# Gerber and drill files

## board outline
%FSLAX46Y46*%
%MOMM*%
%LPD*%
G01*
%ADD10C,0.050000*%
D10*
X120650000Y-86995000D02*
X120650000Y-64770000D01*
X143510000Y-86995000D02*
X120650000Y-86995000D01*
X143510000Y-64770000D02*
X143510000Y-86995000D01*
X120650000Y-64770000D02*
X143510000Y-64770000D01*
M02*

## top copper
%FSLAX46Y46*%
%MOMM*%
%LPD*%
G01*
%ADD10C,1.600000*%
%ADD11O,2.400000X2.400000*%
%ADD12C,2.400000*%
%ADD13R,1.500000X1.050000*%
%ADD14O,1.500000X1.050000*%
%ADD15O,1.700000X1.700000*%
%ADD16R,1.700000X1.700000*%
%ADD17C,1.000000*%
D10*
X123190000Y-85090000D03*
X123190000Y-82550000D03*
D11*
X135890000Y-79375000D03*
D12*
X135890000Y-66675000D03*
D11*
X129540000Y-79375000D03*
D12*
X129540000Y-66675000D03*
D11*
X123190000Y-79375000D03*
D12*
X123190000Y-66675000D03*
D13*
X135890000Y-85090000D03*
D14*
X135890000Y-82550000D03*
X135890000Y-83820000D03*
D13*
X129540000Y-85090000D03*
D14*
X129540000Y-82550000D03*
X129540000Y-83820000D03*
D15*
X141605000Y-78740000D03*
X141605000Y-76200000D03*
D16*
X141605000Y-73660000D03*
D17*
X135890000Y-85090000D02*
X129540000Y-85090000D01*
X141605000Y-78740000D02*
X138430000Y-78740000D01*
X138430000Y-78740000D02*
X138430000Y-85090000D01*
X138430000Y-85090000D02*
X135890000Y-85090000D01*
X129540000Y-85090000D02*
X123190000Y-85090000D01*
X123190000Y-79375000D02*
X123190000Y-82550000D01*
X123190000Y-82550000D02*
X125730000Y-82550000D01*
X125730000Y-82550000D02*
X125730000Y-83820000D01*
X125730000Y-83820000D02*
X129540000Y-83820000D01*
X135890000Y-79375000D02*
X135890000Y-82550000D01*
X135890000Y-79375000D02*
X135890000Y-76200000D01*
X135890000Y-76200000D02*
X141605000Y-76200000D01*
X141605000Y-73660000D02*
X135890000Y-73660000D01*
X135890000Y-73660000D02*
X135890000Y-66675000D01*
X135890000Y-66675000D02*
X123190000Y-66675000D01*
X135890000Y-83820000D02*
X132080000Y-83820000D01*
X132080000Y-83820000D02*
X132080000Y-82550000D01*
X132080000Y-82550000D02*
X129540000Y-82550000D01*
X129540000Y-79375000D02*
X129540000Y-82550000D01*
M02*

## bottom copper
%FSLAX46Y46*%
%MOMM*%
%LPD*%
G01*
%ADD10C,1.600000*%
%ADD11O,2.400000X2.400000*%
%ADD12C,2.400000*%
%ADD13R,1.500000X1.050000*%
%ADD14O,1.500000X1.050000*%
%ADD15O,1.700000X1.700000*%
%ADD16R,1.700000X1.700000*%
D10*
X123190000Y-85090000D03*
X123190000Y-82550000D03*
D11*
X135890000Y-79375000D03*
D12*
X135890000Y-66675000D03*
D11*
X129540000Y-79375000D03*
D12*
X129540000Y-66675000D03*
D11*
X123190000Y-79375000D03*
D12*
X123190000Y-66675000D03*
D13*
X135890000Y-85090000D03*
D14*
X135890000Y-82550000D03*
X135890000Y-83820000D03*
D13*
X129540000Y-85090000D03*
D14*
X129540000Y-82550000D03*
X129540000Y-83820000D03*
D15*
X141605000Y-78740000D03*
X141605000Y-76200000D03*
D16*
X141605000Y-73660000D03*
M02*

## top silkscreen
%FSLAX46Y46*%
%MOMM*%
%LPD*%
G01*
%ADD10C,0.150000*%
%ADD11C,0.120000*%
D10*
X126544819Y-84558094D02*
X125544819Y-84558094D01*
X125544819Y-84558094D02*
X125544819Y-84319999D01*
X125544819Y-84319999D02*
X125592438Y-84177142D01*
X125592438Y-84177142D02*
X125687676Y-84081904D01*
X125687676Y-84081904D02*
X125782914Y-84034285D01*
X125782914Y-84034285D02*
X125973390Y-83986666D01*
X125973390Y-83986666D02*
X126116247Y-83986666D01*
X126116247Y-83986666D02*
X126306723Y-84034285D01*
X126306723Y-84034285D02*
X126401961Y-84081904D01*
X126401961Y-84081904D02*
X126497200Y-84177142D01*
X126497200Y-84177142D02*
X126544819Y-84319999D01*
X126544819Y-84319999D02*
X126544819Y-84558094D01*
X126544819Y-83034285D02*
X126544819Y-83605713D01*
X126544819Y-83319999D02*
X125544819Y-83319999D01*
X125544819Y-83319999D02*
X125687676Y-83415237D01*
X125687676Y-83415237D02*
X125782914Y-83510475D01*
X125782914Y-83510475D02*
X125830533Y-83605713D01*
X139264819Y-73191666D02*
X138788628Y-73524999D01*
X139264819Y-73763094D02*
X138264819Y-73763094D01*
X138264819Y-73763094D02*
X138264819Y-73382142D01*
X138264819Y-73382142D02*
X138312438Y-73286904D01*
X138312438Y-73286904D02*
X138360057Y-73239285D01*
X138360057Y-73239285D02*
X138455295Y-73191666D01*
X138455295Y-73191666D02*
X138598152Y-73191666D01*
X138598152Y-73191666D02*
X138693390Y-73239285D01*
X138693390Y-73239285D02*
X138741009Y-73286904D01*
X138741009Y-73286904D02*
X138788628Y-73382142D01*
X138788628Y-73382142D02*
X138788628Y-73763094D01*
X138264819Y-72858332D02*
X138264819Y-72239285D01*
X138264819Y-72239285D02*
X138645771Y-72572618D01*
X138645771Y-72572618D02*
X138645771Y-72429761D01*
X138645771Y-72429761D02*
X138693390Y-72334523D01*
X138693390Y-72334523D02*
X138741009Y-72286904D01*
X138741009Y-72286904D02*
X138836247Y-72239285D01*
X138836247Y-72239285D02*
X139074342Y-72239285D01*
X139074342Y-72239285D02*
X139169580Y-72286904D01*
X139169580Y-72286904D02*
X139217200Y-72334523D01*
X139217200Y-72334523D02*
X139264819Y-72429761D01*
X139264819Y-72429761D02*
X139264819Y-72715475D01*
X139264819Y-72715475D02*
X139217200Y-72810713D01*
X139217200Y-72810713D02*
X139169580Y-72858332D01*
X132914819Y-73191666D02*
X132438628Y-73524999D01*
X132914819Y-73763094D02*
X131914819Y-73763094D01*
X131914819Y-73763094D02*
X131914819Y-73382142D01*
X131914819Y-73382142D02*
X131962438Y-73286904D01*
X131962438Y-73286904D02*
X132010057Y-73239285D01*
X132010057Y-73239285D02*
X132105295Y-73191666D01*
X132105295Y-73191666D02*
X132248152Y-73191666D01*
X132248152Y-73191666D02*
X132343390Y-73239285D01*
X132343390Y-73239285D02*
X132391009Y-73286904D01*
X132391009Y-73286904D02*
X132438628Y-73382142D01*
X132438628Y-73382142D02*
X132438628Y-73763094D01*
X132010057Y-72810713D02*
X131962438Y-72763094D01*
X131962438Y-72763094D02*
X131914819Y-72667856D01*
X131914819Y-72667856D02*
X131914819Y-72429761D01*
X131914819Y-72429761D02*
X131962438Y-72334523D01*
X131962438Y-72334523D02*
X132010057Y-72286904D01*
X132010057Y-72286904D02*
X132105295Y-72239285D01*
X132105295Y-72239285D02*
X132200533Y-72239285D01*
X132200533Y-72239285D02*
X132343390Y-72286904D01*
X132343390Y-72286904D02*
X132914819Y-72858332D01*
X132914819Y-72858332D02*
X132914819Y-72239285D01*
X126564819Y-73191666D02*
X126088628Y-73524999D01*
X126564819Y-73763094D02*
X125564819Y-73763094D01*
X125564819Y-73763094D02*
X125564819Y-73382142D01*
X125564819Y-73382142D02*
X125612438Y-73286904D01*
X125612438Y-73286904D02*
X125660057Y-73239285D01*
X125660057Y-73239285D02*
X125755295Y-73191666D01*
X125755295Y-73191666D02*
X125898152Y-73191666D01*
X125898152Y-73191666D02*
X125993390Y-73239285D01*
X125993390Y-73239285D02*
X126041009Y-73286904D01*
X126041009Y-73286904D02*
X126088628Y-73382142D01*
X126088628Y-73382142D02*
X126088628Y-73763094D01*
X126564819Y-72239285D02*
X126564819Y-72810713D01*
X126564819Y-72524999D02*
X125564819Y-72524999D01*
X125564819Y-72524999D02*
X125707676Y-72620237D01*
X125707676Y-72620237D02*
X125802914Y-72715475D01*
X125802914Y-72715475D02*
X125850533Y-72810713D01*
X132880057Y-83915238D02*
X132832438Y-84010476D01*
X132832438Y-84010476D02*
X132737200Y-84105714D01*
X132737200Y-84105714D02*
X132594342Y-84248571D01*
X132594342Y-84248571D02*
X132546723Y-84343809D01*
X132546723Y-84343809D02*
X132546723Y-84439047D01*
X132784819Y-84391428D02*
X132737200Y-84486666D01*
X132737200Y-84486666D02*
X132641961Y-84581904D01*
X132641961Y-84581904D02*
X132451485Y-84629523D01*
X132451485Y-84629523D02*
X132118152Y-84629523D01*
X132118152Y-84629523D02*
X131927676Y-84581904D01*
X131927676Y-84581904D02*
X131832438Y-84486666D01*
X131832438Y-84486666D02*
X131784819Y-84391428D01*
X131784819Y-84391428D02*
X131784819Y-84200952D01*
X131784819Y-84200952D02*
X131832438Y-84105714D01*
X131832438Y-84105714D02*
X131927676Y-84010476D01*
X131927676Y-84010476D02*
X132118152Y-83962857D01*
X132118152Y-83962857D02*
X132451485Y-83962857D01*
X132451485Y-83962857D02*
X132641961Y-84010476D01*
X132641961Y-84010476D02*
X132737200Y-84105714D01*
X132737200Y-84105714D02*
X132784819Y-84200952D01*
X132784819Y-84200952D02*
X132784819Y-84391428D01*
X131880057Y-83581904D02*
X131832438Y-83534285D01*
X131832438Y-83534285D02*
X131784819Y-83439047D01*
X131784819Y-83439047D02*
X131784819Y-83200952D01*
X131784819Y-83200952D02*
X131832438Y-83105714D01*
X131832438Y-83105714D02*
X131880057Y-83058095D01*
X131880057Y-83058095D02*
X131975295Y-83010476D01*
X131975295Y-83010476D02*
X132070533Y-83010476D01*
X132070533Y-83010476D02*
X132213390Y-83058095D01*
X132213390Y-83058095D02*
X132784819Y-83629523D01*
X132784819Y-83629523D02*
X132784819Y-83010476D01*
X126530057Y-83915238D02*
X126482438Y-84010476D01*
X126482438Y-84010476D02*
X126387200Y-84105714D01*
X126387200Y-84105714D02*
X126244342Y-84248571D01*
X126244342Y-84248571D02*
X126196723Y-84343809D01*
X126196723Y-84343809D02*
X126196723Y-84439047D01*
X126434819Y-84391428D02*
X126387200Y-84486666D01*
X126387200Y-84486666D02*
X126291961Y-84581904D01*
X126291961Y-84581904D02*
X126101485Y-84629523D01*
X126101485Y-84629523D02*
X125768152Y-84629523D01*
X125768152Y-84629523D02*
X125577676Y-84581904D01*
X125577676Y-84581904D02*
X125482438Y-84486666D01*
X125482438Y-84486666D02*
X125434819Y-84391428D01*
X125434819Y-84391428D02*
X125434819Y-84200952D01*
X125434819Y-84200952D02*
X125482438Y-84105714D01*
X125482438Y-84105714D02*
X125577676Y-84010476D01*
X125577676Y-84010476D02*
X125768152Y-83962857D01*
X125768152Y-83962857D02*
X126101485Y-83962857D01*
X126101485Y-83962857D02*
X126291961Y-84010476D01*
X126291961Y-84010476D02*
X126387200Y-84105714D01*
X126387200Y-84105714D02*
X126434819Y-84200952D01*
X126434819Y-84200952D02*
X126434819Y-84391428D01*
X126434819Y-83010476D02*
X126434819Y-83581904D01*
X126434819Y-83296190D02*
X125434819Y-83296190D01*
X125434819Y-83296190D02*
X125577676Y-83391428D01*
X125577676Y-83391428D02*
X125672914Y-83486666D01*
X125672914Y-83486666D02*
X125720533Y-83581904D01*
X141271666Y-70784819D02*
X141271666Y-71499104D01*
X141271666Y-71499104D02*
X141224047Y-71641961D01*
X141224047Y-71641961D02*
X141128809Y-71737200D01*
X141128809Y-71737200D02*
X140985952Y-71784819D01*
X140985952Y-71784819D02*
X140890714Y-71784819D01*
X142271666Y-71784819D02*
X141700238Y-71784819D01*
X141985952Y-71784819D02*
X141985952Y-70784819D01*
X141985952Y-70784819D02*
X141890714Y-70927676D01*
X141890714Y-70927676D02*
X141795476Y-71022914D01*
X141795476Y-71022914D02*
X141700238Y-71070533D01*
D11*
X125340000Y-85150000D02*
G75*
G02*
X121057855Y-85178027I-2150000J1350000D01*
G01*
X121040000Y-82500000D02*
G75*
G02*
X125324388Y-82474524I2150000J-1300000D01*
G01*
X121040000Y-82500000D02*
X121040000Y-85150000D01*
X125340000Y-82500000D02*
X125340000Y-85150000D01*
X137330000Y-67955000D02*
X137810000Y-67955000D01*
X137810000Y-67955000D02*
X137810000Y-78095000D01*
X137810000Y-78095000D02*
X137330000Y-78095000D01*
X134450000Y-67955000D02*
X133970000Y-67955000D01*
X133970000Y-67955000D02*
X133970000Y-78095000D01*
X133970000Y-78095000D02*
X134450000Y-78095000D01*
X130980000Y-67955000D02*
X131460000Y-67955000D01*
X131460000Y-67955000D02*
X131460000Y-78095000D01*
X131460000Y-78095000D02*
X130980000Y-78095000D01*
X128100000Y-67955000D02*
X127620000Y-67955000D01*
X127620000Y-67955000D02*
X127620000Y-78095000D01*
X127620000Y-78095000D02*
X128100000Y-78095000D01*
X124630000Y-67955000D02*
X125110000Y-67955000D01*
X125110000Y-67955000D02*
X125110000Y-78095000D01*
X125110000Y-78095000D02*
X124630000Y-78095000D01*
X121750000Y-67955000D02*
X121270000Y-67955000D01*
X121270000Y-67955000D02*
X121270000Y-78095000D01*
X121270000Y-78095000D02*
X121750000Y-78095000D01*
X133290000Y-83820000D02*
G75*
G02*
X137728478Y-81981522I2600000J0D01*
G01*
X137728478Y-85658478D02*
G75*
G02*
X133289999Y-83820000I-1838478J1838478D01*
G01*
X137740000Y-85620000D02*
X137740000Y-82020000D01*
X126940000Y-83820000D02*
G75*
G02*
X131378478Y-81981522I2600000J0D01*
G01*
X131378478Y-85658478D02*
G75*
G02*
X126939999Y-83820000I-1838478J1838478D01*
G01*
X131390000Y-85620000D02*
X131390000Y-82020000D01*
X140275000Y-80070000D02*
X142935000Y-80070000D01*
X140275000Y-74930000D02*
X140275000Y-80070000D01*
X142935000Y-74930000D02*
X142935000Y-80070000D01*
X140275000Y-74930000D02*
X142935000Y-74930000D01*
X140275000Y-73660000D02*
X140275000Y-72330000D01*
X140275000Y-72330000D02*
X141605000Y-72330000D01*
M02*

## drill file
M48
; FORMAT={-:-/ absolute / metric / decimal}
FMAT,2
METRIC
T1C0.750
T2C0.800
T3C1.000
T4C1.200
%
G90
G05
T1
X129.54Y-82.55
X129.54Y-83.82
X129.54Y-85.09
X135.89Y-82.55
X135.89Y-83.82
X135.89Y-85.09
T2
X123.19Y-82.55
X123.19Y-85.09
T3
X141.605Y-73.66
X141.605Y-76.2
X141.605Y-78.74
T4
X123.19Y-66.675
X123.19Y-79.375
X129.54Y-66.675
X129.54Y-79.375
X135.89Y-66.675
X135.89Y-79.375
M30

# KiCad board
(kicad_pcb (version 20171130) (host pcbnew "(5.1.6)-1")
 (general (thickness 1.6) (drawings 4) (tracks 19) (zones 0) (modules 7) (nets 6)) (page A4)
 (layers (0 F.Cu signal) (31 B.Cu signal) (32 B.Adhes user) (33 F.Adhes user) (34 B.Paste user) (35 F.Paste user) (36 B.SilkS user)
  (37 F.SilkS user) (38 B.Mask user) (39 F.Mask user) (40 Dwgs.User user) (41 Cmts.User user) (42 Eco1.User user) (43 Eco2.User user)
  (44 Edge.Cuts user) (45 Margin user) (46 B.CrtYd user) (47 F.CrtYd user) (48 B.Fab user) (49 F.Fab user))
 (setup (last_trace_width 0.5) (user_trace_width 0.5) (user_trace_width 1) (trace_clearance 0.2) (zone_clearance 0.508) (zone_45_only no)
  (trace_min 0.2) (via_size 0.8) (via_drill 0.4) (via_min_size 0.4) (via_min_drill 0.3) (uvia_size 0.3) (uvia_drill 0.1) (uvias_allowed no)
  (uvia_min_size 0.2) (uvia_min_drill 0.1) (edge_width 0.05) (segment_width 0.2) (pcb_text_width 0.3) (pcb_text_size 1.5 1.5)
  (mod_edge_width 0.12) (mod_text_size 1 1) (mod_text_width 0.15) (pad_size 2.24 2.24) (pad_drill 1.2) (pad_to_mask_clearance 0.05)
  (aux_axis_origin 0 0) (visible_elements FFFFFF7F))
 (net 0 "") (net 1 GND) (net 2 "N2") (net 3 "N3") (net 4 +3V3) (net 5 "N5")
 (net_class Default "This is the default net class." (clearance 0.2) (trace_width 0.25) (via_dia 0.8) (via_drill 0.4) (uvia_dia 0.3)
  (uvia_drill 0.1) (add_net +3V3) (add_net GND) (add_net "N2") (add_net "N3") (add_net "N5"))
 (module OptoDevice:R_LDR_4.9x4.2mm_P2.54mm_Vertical (layer F.Cu) (at 123.19 82.55 270)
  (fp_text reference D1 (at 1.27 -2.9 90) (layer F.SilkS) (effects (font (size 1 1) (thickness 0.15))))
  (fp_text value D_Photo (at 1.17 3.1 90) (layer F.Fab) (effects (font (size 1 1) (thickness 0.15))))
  (fp_arc (start 1.25 0) (end 2.6 -2.15) (angle 115) (layer F.SilkS) (width 0.12))
  (fp_arc (start 1.25 0) (end -0.05 2.15) (angle 117) (layer F.SilkS) (width 0.12))
  (fp_line (start -0.05 2.15) (end 2.6 2.15) (layer F.SilkS) (width 0.12))
  (fp_line (start -0.05 -2.15) (end 2.6 -2.15) (layer F.SilkS) (width 0.12))
  (pad 2 thru_hole circle (at 2.54 0 270) (size 1.6 1.6) (drill 0.8) (layers *.Cu *.Mask) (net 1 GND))
  (pad 1 thru_hole circle (at 0 0 270) (size 1.6 1.6) (drill 0.8) (layers *.Cu *.Mask) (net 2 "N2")))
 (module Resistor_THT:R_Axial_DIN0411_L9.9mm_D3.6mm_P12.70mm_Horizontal (layer F.Cu) (at 135.89 66.675 270)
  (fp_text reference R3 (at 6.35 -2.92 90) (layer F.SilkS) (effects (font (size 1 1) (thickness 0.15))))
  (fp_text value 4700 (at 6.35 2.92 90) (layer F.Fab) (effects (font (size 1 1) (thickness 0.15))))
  (fp_line (start 1.28 -1.44) (end 1.28 -1.92) (layer F.SilkS) (width 0.12))
  (fp_line (start 1.28 -1.92) (end 11.42 -1.92) (layer F.SilkS) (width 0.12))
  (fp_line (start 11.42 -1.92) (end 11.42 -1.44) (layer F.SilkS) (width 0.12))
  (fp_line (start 1.28 1.44) (end 1.28 1.92) (layer F.SilkS) (width 0.12))
  (fp_line (start 1.28 1.92) (end 11.42 1.92) (layer F.SilkS) (width 0.12))
  (fp_line (start 11.42 1.92) (end 11.42 1.44) (layer F.SilkS) (width 0.12))
  (pad 2 thru_hole oval (at 12.7 0 270) (size 2.4 2.4) (drill 1.2) (layers *.Cu *.Mask) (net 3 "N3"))
  (pad 1 thru_hole circle (at 0 0 270) (size 2.4 2.4) (drill 1.2) (layers *.Cu *.Mask) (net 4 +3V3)))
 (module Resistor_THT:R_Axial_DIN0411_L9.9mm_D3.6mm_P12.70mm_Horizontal (layer F.Cu) (at 129.54 66.675 270)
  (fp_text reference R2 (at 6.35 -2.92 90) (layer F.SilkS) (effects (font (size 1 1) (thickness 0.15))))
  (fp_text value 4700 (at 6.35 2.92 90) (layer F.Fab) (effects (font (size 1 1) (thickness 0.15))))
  (fp_line (start 1.28 -1.44) (end 1.28 -1.92) (layer F.SilkS) (width 0.12))
  (fp_line (start 1.28 -1.92) (end 11.42 -1.92) (layer F.SilkS) (width 0.12))
  (fp_line (start 11.42 -1.92) (end 11.42 -1.44) (layer F.SilkS) (width 0.12))
  (fp_line (start 1.28 1.44) (end 1.28 1.92) (layer F.SilkS) (width 0.12))
  (fp_line (start 1.28 1.92) (end 11.42 1.92) (layer F.SilkS) (width 0.12))
  (fp_line (start 11.42 1.92) (end 11.42 1.44) (layer F.SilkS) (width 0.12))
  (pad 2 thru_hole oval (at 12.7 0 270) (size 2.4 2.4) (drill 1.2) (layers *.Cu *.Mask) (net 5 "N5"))
  (pad 1 thru_hole circle (at 0 0 270) (size 2.4 2.4) (drill 1.2) (layers *.Cu *.Mask) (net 4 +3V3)))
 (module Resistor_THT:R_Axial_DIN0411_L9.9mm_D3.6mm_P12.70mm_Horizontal (layer F.Cu) (at 123.19 66.675 270)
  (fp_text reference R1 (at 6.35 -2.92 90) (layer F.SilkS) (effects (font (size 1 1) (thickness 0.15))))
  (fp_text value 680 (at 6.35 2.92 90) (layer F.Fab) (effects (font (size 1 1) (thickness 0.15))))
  (fp_line (start 1.28 -1.44) (end 1.28 -1.92) (layer F.SilkS) (width 0.12))
  (fp_line (start 1.28 -1.92) (end 11.42 -1.92) (layer F.SilkS) (width 0.12))
  (fp_line (start 11.42 -1.92) (end 11.42 -1.44) (layer F.SilkS) (width 0.12))
  (fp_line (start 1.28 1.44) (end 1.28 1.92) (layer F.SilkS) (width 0.12))
  (fp_line (start 1.28 1.92) (end 11.42 1.92) (layer F.SilkS) (width 0.12))
  (fp_line (start 11.42 1.92) (end 11.42 1.44) (layer F.SilkS) (width 0.12))
  (pad 2 thru_hole oval (at 12.7 0 270) (size 2.4 2.4) (drill 1.2) (layers *.Cu *.Mask) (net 2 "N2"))
  (pad 1 thru_hole circle (at 0 0 270) (size 2.4 2.4) (drill 1.2) (layers *.Cu *.Mask) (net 4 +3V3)))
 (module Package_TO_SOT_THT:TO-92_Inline (layer F.Cu) (at 135.89 85.09 90)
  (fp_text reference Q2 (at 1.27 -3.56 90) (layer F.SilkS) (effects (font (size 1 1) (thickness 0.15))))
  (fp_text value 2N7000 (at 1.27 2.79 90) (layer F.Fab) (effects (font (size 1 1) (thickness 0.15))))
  (fp_arc (start 1.27 0) (end 1.27 -2.6) (angle 135) (layer F.SilkS) (width 0.12))
  (fp_arc (start 1.27 0) (end 1.27 -2.6) (angle -135) (layer F.SilkS) (width 0.12))
  (fp_line (start -0.53 1.85) (end 3.07 1.85) (layer F.SilkS) (width 0.12))
  (pad 1 thru_hole rect (at 0 0 90) (size 1.05 1.5) (drill 0.75) (layers *.Cu *.Mask) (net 1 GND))
  (pad 3 thru_hole oval (at 2.54 0 90) (size 1.05 1.5) (drill 0.75) (layers *.Cu *.Mask) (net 3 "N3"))
  (pad 2 thru_hole oval (at 1.27 0 90) (size 1.05 1.5) (drill 0.75) (layers *.Cu *.Mask) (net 5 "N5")))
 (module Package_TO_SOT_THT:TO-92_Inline (layer F.Cu) (at 129.54 85.09 90)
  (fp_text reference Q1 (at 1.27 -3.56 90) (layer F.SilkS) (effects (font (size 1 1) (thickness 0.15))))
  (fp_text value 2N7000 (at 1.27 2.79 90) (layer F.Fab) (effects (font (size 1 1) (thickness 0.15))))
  (fp_arc (start 1.27 0) (end 1.27 -2.6) (angle 135) (layer F.SilkS) (width 0.12))
  (fp_arc (start 1.27 0) (end 1.27 -2.6) (angle -135) (layer F.SilkS) (width 0.12))
  (fp_line (start -0.53 1.85) (end 3.07 1.85) (layer F.SilkS) (width 0.12))
  (pad 1 thru_hole rect (at 0 0 90) (size 1.05 1.5) (drill 0.75) (layers *.Cu *.Mask) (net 1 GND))
  (pad 3 thru_hole oval (at 2.54 0 90) (size 1.05 1.5) (drill 0.75) (layers *.Cu *.Mask) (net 5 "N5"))
  (pad 2 thru_hole oval (at 1.27 0 90) (size 1.05 1.5) (drill 0.75) (layers *.Cu *.Mask) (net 2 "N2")))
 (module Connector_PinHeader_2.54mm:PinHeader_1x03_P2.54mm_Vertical (layer F.Cu) (at 141.605 73.66)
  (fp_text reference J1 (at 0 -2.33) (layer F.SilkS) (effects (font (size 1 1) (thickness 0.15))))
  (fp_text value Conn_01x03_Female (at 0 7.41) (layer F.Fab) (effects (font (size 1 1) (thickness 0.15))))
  (fp_line (start -1.33 6.41) (end 1.33 6.41) (layer F.SilkS) (width 0.12))
  (fp_line (start -1.33 1.27) (end -1.33 6.41) (layer F.SilkS) (width 0.12))
  (fp_line (start 1.33 1.27) (end 1.33 6.41) (layer F.SilkS) (width 0.12))
  (fp_line (start -1.33 1.27) (end 1.33 1.27) (layer F.SilkS) (width 0.12))
  (fp_line (start -1.33 0) (end -1.33 -1.33) (layer F.SilkS) (width 0.12))
  (fp_line (start -1.33 -1.33) (end 0 -1.33) (layer F.SilkS) (width 0.12))
  (pad 3 thru_hole oval (at 0 5.08) (size 1.7 1.7) (drill 1) (layers *.Cu *.Mask) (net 1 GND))
  (pad 2 thru_hole oval (at 0 2.54) (size 1.7 1.7) (drill 1) (layers *.Cu *.Mask) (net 3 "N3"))
  (pad 1 thru_hole rect (at 0 0) (size 1.7 1.7) (drill 1) (layers *.Cu *.Mask) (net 4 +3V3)))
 (gr_line (start 120.65 86.995) (end 120.65 64.77) (layer Edge.Cuts) (width 0.05))
 (gr_line (start 143.51 86.995) (end 120.65 86.995) (layer Edge.Cuts) (width 0.05))
 (gr_line (start 143.51 64.77) (end 143.51 86.995) (layer Edge.Cuts) (width 0.05))
 (gr_line (start 120.65 64.77) (end 143.51 64.77) (layer Edge.Cuts) (width 0.05))
 (segment (start 135.89 85.09) (end 129.54 85.09) (width 1) (layer F.Cu) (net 1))
 (segment (start 141.605 78.74) (end 138.43 78.74) (width 1) (layer F.Cu) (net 1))
 (segment (start 138.43 78.74) (end 138.43 85.09) (width 1) (layer F.Cu) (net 1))
 (segment (start 138.43 85.09) (end 135.89 85.09) (width 1) (layer F.Cu) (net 1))
 (segment (start 129.54 85.09) (end 123.19 85.09) (width 1) (layer F.Cu) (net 1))
 (segment (start 123.19 79.375) (end 123.19 82.55) (width 1) (layer F.Cu) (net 2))
 (segment (start 123.19 82.55) (end 125.73 82.55) (width 1) (layer F.Cu) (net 2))
 (segment (start 125.73 82.55) (end 125.73 83.82) (width 1) (layer F.Cu) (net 2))
 (segment (start 125.73 83.82) (end 129.54 83.82) (width 1) (layer F.Cu) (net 2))
 (segment (start 135.89 79.375) (end 135.89 82.55) (width 1) (layer F.Cu) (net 3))
 (segment (start 135.89 79.375) (end 135.89 76.2) (width 1) (layer F.Cu) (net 3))
 (segment (start 135.89 76.2) (end 141.605 76.2) (width 1) (layer F.Cu) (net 3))
 (segment (start 141.605 73.66) (end 135.89 73.66) (width 1) (layer F.Cu) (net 4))
 (segment (start 135.89 73.66) (end 135.89 66.675) (width 1) (layer F.Cu) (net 4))
 (segment (start 135.89 66.675) (end 123.19 66.675) (width 1) (layer F.Cu) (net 4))
 (segment (start 135.89 83.82) (end 132.08 83.82) (width 1) (layer F.Cu) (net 5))
 (segment (start 132.08 83.82) (end 132.08 82.55) (width 1) (layer F.Cu) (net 5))
 (segment (start 132.08 82.55) (end 129.54 82.55) (width 1) (layer F.Cu) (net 5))
 (segment (start 129.54 79.375) (end 129.54 82.55) (width 1) (layer F.Cu) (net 5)))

